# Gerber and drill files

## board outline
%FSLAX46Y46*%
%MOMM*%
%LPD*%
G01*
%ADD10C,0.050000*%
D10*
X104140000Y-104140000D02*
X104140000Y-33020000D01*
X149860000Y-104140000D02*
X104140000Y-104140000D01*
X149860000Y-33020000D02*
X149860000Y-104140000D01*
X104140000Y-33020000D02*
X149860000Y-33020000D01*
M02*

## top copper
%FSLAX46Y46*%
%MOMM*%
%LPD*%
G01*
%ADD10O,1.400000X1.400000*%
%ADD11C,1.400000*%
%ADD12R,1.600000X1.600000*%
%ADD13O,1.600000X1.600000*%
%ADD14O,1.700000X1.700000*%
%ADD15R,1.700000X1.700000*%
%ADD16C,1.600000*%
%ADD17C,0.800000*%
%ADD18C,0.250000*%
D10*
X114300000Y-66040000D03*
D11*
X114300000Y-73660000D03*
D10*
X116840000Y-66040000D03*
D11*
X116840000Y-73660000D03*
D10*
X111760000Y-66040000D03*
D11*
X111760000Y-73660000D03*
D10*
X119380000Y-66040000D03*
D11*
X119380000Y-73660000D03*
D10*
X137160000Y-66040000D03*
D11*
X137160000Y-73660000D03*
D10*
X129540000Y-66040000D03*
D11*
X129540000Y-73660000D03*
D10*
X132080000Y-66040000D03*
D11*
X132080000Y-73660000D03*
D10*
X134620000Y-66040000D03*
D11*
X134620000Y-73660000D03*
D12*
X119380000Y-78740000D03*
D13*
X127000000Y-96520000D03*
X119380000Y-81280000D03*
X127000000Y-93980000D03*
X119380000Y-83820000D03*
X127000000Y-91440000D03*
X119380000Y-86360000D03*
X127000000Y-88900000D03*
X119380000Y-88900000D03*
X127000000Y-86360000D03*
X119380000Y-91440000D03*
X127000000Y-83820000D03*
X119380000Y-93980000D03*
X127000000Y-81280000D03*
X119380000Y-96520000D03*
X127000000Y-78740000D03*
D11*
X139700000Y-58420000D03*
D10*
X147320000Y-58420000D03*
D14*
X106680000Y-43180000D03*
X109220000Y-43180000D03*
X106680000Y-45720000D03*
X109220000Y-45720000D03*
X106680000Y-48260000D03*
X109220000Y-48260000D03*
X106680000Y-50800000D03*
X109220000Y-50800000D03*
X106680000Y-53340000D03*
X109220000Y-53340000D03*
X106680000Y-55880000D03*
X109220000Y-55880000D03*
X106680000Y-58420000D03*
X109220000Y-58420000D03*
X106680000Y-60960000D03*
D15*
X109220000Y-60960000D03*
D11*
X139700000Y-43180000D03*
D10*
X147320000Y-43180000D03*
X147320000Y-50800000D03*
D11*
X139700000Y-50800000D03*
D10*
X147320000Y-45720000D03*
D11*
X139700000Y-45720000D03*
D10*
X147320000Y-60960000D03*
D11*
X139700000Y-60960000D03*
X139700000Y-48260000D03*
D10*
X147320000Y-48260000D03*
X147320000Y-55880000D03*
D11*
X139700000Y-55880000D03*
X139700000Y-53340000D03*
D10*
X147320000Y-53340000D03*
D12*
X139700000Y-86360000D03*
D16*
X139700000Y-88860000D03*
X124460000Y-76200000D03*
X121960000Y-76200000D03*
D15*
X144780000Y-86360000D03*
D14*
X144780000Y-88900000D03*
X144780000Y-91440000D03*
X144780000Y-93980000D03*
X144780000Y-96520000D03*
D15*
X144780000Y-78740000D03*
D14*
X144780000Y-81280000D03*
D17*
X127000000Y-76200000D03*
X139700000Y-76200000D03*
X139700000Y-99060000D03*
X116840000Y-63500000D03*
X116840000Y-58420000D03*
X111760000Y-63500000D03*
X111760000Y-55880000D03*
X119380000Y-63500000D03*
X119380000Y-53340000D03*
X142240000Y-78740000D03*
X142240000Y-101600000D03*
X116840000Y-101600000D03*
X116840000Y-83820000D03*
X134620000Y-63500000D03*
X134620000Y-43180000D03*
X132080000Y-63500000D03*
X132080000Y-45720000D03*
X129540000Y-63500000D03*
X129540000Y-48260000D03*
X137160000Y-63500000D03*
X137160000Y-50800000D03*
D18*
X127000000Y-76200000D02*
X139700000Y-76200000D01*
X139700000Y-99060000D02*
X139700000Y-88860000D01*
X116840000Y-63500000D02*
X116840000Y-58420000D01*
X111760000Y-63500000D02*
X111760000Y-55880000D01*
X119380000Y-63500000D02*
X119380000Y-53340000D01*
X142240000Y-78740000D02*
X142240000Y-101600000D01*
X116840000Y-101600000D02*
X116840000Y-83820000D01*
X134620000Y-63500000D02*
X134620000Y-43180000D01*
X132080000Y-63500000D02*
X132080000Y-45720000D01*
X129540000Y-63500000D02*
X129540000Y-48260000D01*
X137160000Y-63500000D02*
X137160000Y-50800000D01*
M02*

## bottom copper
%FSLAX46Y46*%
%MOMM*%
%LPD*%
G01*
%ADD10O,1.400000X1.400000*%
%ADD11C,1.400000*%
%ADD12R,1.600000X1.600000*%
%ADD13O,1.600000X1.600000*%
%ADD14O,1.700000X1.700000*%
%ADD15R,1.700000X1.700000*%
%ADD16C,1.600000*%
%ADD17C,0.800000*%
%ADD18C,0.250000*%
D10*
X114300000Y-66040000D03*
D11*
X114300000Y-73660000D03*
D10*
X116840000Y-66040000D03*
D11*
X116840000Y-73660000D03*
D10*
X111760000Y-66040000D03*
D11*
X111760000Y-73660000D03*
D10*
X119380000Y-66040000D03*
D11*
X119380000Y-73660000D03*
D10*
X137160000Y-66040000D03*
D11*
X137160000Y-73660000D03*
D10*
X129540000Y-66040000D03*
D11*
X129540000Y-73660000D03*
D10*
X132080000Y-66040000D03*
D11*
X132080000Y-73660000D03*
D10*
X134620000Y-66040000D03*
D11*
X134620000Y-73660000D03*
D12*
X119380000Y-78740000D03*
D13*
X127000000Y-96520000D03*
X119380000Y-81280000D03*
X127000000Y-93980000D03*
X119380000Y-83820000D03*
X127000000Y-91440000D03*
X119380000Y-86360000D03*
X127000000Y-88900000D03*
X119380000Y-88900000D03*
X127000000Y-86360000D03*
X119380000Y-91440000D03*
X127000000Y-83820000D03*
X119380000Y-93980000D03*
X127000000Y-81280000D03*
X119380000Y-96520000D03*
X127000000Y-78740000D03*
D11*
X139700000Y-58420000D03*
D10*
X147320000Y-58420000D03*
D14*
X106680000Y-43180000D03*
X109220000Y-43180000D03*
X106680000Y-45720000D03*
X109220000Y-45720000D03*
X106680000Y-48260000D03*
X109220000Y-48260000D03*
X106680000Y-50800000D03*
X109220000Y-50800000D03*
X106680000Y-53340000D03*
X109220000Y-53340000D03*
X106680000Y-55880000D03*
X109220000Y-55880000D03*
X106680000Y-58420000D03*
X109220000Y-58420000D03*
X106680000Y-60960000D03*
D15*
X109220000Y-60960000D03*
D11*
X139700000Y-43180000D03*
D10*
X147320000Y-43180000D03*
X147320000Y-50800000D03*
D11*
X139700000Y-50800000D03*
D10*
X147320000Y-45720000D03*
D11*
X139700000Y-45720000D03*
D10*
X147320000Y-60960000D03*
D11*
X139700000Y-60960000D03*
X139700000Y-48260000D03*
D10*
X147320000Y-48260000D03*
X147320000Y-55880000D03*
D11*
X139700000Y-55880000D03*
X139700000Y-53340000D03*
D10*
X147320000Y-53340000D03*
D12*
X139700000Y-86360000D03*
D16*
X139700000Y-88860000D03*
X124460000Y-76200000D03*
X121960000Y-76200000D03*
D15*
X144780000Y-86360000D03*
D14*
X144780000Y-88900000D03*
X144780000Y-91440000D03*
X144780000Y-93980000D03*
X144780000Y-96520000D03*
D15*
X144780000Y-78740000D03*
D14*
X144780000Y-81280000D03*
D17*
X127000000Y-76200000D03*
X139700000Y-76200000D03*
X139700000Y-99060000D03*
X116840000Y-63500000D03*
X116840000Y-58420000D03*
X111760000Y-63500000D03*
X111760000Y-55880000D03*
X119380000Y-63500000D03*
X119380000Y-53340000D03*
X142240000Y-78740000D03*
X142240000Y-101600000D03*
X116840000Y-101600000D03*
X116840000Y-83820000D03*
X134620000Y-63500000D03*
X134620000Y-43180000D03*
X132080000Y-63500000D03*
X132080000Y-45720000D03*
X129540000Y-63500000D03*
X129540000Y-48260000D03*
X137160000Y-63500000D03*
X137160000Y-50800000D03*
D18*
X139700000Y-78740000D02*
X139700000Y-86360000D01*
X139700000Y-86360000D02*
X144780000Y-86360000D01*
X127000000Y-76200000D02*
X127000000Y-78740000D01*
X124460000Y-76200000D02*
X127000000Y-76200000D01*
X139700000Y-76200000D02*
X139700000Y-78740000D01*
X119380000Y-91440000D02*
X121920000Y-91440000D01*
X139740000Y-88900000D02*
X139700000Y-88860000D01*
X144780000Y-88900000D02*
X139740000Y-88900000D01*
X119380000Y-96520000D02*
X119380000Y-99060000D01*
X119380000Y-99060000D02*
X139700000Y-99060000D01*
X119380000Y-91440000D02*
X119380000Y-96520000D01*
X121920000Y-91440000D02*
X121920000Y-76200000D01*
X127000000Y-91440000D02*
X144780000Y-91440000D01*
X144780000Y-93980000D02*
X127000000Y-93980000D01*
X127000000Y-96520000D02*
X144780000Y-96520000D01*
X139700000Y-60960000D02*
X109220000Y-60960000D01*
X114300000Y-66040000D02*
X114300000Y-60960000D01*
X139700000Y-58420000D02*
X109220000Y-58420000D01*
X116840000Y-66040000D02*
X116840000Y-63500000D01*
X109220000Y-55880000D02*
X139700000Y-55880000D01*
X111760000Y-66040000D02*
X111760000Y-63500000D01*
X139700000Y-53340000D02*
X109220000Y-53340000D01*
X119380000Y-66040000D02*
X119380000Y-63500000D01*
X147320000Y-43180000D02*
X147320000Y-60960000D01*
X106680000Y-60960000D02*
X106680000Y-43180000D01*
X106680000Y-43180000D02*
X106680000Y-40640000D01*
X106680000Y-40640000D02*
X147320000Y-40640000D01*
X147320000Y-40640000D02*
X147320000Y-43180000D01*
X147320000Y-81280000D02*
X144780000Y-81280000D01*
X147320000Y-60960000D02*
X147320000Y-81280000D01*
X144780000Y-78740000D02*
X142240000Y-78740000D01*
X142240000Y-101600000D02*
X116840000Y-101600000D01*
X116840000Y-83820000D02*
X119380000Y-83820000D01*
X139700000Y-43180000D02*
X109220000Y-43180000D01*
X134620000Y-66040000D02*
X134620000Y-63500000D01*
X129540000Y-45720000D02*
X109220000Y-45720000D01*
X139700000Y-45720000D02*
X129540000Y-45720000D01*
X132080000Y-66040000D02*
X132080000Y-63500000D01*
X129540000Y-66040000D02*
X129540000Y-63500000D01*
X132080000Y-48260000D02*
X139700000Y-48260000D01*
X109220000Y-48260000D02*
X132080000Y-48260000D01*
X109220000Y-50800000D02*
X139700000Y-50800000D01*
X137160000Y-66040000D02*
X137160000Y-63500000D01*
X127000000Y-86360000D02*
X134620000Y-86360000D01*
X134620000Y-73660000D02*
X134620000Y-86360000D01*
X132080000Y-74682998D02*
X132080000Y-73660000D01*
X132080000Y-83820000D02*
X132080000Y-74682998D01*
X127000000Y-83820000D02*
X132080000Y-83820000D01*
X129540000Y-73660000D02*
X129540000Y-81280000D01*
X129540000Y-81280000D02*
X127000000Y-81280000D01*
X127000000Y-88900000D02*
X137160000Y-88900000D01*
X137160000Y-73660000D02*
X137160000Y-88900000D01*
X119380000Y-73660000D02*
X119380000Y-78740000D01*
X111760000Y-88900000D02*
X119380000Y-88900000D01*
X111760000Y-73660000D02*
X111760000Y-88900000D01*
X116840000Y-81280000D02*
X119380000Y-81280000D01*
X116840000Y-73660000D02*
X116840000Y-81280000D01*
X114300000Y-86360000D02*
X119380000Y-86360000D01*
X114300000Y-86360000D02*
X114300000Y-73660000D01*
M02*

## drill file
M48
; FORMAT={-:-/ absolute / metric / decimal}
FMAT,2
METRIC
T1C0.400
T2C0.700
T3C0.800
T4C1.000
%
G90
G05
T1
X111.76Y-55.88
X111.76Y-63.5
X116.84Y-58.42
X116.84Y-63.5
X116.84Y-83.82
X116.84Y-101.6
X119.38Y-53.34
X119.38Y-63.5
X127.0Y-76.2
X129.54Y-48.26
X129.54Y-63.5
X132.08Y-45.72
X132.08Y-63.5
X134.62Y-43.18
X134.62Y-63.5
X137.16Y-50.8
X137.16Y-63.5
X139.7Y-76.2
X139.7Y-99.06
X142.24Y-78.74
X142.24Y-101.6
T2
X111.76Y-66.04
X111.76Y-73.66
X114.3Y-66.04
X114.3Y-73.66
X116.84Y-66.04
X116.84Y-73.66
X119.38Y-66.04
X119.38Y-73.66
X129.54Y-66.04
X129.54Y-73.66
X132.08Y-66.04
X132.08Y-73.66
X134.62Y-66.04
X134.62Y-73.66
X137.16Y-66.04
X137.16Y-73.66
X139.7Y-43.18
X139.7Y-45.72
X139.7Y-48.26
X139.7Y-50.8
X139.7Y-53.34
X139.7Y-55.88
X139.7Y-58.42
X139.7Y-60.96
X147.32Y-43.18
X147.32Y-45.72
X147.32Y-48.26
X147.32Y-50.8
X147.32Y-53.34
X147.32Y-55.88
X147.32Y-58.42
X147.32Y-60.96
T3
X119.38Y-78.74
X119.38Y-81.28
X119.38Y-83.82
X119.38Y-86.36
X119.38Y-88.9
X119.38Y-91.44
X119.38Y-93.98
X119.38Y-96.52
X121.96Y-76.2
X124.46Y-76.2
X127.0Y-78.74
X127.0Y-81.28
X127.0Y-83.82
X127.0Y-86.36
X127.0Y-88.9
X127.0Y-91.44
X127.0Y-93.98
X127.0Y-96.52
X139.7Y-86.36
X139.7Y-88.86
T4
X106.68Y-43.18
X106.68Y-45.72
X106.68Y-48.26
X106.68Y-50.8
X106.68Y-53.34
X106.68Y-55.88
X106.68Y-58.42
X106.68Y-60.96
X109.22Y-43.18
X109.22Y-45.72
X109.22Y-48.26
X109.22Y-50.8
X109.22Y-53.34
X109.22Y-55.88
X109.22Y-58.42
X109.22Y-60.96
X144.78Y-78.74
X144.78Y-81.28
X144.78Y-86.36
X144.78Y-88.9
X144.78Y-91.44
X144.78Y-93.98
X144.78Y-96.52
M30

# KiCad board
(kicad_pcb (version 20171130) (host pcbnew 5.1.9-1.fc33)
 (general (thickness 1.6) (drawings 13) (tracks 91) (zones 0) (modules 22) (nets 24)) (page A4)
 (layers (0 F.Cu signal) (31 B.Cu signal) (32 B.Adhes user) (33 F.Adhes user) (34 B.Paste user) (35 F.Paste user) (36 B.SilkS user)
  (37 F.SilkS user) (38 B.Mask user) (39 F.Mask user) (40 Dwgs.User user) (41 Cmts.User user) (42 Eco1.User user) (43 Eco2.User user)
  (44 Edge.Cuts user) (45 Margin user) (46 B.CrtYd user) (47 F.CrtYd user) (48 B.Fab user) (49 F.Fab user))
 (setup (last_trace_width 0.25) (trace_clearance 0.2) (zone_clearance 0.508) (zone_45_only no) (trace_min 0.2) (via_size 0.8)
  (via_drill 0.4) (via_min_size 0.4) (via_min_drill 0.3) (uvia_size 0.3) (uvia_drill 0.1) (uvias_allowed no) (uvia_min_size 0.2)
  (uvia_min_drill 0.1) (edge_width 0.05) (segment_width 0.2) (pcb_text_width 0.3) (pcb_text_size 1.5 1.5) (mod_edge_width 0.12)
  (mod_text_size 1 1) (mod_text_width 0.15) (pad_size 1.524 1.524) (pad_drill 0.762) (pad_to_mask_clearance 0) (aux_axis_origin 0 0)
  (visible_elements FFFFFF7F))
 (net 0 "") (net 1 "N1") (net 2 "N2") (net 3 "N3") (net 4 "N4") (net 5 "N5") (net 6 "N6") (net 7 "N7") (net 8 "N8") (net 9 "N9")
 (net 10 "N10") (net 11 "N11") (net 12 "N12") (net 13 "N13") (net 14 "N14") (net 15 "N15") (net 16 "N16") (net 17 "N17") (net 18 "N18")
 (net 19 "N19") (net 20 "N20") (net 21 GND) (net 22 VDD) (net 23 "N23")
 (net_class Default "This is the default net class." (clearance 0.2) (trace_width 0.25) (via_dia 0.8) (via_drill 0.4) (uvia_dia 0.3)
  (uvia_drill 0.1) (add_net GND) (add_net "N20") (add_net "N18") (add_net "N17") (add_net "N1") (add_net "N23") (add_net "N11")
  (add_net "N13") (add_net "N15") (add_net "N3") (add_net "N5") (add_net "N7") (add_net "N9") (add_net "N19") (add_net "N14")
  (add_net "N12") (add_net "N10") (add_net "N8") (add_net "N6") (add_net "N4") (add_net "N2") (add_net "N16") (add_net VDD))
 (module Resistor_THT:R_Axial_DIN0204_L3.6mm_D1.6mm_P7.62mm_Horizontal (layer F.Cu) (at 114.3 73.66 90)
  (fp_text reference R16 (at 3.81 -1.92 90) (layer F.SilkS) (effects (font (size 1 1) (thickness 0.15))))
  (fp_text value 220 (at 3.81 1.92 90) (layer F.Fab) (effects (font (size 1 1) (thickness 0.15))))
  (pad 2 thru_hole oval (at 7.62 0 90) (size 1.4 1.4) (drill 0.7) (layers *.Cu *.Mask) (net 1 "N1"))
  (pad 1 thru_hole circle (at 0 0 90) (size 1.4 1.4) (drill 0.7) (layers *.Cu *.Mask) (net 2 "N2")))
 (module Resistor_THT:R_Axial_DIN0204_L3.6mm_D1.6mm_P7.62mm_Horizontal (layer F.Cu) (at 116.84 73.66 90)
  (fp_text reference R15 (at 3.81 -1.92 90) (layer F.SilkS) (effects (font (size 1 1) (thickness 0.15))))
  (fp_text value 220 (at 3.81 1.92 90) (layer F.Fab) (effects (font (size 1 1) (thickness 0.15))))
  (pad 2 thru_hole oval (at 7.62 0 90) (size 1.4 1.4) (drill 0.7) (layers *.Cu *.Mask) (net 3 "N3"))
  (pad 1 thru_hole circle (at 0 0 90) (size 1.4 1.4) (drill 0.7) (layers *.Cu *.Mask) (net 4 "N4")))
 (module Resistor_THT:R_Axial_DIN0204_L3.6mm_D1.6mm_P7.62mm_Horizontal (layer F.Cu) (at 111.76 73.66 90)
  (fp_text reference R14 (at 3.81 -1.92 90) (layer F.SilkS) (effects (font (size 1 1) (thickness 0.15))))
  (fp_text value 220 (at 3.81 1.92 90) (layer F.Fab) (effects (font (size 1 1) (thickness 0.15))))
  (pad 2 thru_hole oval (at 7.62 0 90) (size 1.4 1.4) (drill 0.7) (layers *.Cu *.Mask) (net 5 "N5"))
  (pad 1 thru_hole circle (at 0 0 90) (size 1.4 1.4) (drill 0.7) (layers *.Cu *.Mask) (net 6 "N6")))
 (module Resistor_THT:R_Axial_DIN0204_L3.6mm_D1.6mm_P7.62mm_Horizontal (layer F.Cu) (at 119.38 73.66 90)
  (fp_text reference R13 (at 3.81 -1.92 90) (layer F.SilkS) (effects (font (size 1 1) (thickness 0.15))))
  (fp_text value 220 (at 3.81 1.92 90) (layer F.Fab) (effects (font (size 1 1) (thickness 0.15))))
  (pad 2 thru_hole oval (at 7.62 0 90) (size 1.4 1.4) (drill 0.7) (layers *.Cu *.Mask) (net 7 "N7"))
  (pad 1 thru_hole circle (at 0 0 90) (size 1.4 1.4) (drill 0.7) (layers *.Cu *.Mask) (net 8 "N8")))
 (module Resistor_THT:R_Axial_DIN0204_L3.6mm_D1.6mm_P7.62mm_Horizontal (layer F.Cu) (at 137.16 73.66 90)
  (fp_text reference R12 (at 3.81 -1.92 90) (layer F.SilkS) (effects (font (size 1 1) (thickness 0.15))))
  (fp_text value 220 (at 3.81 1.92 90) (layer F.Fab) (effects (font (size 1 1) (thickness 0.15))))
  (pad 2 thru_hole oval (at 7.62 0 90) (size 1.4 1.4) (drill 0.7) (layers *.Cu *.Mask) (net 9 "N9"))
  (pad 1 thru_hole circle (at 0 0 90) (size 1.4 1.4) (drill 0.7) (layers *.Cu *.Mask) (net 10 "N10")))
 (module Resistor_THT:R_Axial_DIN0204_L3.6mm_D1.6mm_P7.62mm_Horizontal (layer F.Cu) (at 129.54 73.66 90)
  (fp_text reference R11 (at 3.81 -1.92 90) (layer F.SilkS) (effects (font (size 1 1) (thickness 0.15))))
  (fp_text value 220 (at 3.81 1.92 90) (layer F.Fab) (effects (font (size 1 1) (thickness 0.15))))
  (pad 2 thru_hole oval (at 7.62 0 90) (size 1.4 1.4) (drill 0.7) (layers *.Cu *.Mask) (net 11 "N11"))
  (pad 1 thru_hole circle (at 0 0 90) (size 1.4 1.4) (drill 0.7) (layers *.Cu *.Mask) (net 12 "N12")))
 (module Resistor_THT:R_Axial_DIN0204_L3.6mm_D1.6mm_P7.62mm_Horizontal (layer F.Cu) (at 132.08 73.66 90)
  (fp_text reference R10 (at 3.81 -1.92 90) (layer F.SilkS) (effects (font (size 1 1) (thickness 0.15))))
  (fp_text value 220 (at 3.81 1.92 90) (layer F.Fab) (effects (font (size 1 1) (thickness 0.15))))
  (pad 2 thru_hole oval (at 7.62 0 90) (size 1.4 1.4) (drill 0.7) (layers *.Cu *.Mask) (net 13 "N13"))
  (pad 1 thru_hole circle (at 0 0 90) (size 1.4 1.4) (drill 0.7) (layers *.Cu *.Mask) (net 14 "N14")))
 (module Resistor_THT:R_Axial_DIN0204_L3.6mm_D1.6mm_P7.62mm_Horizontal (layer F.Cu) (at 134.62 73.66 90)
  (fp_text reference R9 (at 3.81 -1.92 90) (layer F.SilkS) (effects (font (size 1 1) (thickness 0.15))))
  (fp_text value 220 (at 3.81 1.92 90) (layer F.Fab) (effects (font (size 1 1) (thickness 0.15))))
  (pad 2 thru_hole oval (at 7.62 0 90) (size 1.4 1.4) (drill 0.7) (layers *.Cu *.Mask) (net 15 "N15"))
  (pad 1 thru_hole circle (at 0 0 90) (size 1.4 1.4) (drill 0.7) (layers *.Cu *.Mask) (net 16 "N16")))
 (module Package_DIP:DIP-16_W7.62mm (layer F.Cu) (at 119.38 78.74)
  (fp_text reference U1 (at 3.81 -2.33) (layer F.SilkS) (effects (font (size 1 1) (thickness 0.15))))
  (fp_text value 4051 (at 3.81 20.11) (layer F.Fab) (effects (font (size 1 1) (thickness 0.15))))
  (pad 1 thru_hole rect (at 0 0) (size 1.6 1.6) (drill 0.8) (layers *.Cu *.Mask) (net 8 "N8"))
  (pad 9 thru_hole oval (at 7.62 17.78) (size 1.6 1.6) (drill 0.8) (layers *.Cu *.Mask) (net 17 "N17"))
  (pad 2 thru_hole oval (at 0 2.54) (size 1.6 1.6) (drill 0.8) (layers *.Cu *.Mask) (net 4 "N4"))
  (pad 10 thru_hole oval (at 7.62 15.24) (size 1.6 1.6) (drill 0.8) (layers *.Cu *.Mask) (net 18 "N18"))
  (pad 3 thru_hole oval (at 0 5.08) (size 1.6 1.6) (drill 0.8) (layers *.Cu *.Mask) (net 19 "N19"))
  (pad 11 thru_hole oval (at 7.62 12.7) (size 1.6 1.6) (drill 0.8) (layers *.Cu *.Mask) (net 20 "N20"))
  (pad 4 thru_hole oval (at 0 7.62) (size 1.6 1.6) (drill 0.8) (layers *.Cu *.Mask) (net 2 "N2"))
  (pad 12 thru_hole oval (at 7.62 10.16) (size 1.6 1.6) (drill 0.8) (layers *.Cu *.Mask) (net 10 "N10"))
  (pad 5 thru_hole oval (at 0 10.16) (size 1.6 1.6) (drill 0.8) (layers *.Cu *.Mask) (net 6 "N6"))
  (pad 13 thru_hole oval (at 7.62 7.62) (size 1.6 1.6) (drill 0.8) (layers *.Cu *.Mask) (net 16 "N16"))
  (pad 6 thru_hole oval (at 0 12.7) (size 1.6 1.6) (drill 0.8) (layers *.Cu *.Mask) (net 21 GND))
  (pad 14 thru_hole oval (at 7.62 5.08) (size 1.6 1.6) (drill 0.8) (layers *.Cu *.Mask) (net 14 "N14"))
  (pad 7 thru_hole oval (at 0 15.24) (size 1.6 1.6) (drill 0.8) (layers *.Cu *.Mask) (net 21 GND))
  (pad 15 thru_hole oval (at 7.62 2.54) (size 1.6 1.6) (drill 0.8) (layers *.Cu *.Mask) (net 12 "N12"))
  (pad 8 thru_hole oval (at 0 17.78) (size 1.6 1.6) (drill 0.8) (layers *.Cu *.Mask) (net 21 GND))
  (pad 16 thru_hole oval (at 7.62 0) (size 1.6 1.6) (drill 0.8) (layers *.Cu *.Mask) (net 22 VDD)))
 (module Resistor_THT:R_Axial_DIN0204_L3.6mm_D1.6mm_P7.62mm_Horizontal (layer F.Cu) (at 139.7 58.42)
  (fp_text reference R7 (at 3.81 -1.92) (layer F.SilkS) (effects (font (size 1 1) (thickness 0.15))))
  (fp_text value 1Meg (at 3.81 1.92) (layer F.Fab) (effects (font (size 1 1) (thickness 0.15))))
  (pad 1 thru_hole circle (at 0 0) (size 1.4 1.4) (drill 0.7) (layers *.Cu *.Mask) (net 3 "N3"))
  (pad 2 thru_hole oval (at 7.62 0) (size 1.4 1.4) (drill 0.7) (layers *.Cu *.Mask) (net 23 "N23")))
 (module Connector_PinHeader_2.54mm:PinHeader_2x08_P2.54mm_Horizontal (layer F.Cu) (at 109.22 60.96 180)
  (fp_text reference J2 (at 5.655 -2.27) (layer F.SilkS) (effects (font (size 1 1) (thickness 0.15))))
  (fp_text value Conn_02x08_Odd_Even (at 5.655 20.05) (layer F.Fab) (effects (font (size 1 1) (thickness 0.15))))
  (pad 16 thru_hole oval (at 2.54 17.78 180) (size 1.7 1.7) (drill 1) (layers *.Cu *.Mask) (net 23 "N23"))
  (pad 15 thru_hole oval (at 0 17.78 180) (size 1.7 1.7) (drill 1) (layers *.Cu *.Mask) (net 15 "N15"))
  (pad 14 thru_hole oval (at 2.54 15.24 180) (size 1.7 1.7) (drill 1) (layers *.Cu *.Mask) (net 23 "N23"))
  (pad 13 thru_hole oval (at 0 15.24 180) (size 1.7 1.7) (drill 1) (layers *.Cu *.Mask) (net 13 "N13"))
  (pad 12 thru_hole oval (at 2.54 12.7 180) (size 1.7 1.7) (drill 1) (layers *.Cu *.Mask) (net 23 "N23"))
  (pad 11 thru_hole oval (at 0 12.7 180) (size 1.7 1.7) (drill 1) (layers *.Cu *.Mask) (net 11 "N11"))
  (pad 10 thru_hole oval (at 2.54 10.16 180) (size 1.7 1.7) (drill 1) (layers *.Cu *.Mask) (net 23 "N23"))
  (pad 9 thru_hole oval (at 0 10.16 180) (size 1.7 1.7) (drill 1) (layers *.Cu *.Mask) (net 9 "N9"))
  (pad 8 thru_hole oval (at 2.54 7.62 180) (size 1.7 1.7) (drill 1) (layers *.Cu *.Mask) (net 23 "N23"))
  (pad 7 thru_hole oval (at 0 7.62 180) (size 1.7 1.7) (drill 1) (layers *.Cu *.Mask) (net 7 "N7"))
  (pad 6 thru_hole oval (at 2.54 5.08 180) (size 1.7 1.7) (drill 1) (layers *.Cu *.Mask) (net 23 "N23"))
  (pad 5 thru_hole oval (at 0 5.08 180) (size 1.7 1.7) (drill 1) (layers *.Cu *.Mask) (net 5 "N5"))
  (pad 4 thru_hole oval (at 2.54 2.54 180) (size 1.7 1.7) (drill 1) (layers *.Cu *.Mask) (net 23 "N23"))
  (pad 3 thru_hole oval (at 0 2.54 180) (size 1.7 1.7) (drill 1) (layers *.Cu *.Mask) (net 3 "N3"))
  (pad 2 thru_hole oval (at 2.54 0 180) (size 1.7 1.7) (drill 1) (layers *.Cu *.Mask) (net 23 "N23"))
  (pad 1 thru_hole rect (at 0 0 180) (size 1.7 1.7) (drill 1) (layers *.Cu *.Mask) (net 1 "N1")))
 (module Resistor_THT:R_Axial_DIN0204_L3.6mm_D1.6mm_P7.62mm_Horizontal (layer F.Cu) (at 139.7 43.18)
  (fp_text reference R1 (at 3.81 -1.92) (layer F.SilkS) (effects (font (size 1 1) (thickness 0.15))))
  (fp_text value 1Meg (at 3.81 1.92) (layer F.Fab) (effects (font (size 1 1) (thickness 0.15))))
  (pad 1 thru_hole circle (at 0 0) (size 1.4 1.4) (drill 0.7) (layers *.Cu *.Mask) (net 15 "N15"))
  (pad 2 thru_hole oval (at 7.62 0) (size 1.4 1.4) (drill 0.7) (layers *.Cu *.Mask) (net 23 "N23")))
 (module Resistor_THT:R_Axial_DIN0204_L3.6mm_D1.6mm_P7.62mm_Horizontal (layer F.Cu) (at 139.7 50.8)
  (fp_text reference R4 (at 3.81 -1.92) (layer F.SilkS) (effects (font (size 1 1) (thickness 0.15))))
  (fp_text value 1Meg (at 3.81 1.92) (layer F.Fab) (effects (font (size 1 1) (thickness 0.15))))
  (pad 2 thru_hole oval (at 7.62 0) (size 1.4 1.4) (drill 0.7) (layers *.Cu *.Mask) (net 23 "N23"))
  (pad 1 thru_hole circle (at 0 0) (size 1.4 1.4) (drill 0.7) (layers *.Cu *.Mask) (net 9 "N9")))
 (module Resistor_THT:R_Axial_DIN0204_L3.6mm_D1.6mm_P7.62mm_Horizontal (layer F.Cu) (at 139.7 45.72)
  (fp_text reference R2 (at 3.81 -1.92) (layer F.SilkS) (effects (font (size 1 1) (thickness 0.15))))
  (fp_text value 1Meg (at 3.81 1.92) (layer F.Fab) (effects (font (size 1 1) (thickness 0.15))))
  (pad 2 thru_hole oval (at 7.62 0) (size 1.4 1.4) (drill 0.7) (layers *.Cu *.Mask) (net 23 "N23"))
  (pad 1 thru_hole circle (at 0 0) (size 1.4 1.4) (drill 0.7) (layers *.Cu *.Mask) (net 13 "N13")))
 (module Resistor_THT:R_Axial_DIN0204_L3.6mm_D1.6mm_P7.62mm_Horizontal (layer F.Cu) (at 139.7 60.96)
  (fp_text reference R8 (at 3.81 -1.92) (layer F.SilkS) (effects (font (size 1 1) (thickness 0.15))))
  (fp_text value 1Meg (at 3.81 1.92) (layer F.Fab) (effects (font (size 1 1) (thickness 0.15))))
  (pad 2 thru_hole oval (at 7.62 0) (size 1.4 1.4) (drill 0.7) (layers *.Cu *.Mask) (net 23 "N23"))
  (pad 1 thru_hole circle (at 0 0) (size 1.4 1.4) (drill 0.7) (layers *.Cu *.Mask) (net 1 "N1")))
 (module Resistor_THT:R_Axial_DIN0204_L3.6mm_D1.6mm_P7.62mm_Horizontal (layer F.Cu) (at 139.7 48.26)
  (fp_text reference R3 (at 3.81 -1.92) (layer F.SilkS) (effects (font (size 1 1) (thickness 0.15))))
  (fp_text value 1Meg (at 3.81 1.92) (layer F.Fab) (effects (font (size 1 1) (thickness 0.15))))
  (pad 1 thru_hole circle (at 0 0) (size 1.4 1.4) (drill 0.7) (layers *.Cu *.Mask) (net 11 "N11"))
  (pad 2 thru_hole oval (at 7.62 0) (size 1.4 1.4) (drill 0.7) (layers *.Cu *.Mask) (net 23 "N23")))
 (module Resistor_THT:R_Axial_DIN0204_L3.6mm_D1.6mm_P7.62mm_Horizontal (layer F.Cu) (at 139.7 55.88)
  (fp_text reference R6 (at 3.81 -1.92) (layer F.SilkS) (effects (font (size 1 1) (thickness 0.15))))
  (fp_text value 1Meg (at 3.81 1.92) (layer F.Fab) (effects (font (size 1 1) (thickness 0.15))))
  (pad 2 thru_hole oval (at 7.62 0) (size 1.4 1.4) (drill 0.7) (layers *.Cu *.Mask) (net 23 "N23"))
  (pad 1 thru_hole circle (at 0 0) (size 1.4 1.4) (drill 0.7) (layers *.Cu *.Mask) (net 5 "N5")))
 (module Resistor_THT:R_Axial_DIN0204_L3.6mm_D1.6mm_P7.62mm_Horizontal (layer F.Cu) (at 139.7 53.34)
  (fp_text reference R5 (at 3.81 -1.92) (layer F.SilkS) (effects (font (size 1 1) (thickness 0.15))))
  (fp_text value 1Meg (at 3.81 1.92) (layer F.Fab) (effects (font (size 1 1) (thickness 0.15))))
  (pad 1 thru_hole circle (at 0 0) (size 1.4 1.4) (drill 0.7) (layers *.Cu *.Mask) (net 7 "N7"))
  (pad 2 thru_hole oval (at 7.62 0) (size 1.4 1.4) (drill 0.7) (layers *.Cu *.Mask) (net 23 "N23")))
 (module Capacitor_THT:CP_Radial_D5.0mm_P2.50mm (layer F.Cu) (at 139.7 86.36 270)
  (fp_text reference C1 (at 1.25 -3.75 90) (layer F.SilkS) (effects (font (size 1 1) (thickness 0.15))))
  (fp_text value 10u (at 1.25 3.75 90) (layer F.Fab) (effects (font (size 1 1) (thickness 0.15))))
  (pad 1 thru_hole rect (at 0 0 270) (size 1.6 1.6) (drill 0.8) (layers *.Cu *.Mask) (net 22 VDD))
  (pad 2 thru_hole circle (at 2.5 0 270) (size 1.6 1.6) (drill 0.8) (layers *.Cu *.Mask) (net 21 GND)))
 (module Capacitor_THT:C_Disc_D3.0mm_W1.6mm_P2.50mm (layer F.Cu) (at 124.46 76.2 180)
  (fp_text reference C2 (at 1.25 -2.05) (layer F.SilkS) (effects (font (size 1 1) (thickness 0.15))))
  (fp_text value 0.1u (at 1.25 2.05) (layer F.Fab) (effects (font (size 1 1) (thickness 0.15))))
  (pad 1 thru_hole circle (at 0 0 180) (size 1.6 1.6) (drill 0.8) (layers *.Cu *.Mask) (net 22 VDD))
  (pad 2 thru_hole circle (at 2.5 0 180) (size 1.6 1.6) (drill 0.8) (layers *.Cu *.Mask) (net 21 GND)))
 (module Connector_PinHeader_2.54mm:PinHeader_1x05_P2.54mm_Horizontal (layer F.Cu) (at 144.78 86.36)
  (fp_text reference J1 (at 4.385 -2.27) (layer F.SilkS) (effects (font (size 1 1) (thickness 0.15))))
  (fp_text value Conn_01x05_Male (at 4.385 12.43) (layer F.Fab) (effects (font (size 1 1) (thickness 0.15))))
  (pad 1 thru_hole rect (at 0 0) (size 1.7 1.7) (drill 1) (layers *.Cu *.Mask) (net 22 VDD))
  (pad 2 thru_hole oval (at 0 2.54) (size 1.7 1.7) (drill 1) (layers *.Cu *.Mask) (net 21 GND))
  (pad 3 thru_hole oval (at 0 5.08) (size 1.7 1.7) (drill 1) (layers *.Cu *.Mask) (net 20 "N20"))
  (pad 4 thru_hole oval (at 0 7.62) (size 1.7 1.7) (drill 1) (layers *.Cu *.Mask) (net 18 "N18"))
  (pad 5 thru_hole oval (at 0 10.16) (size 1.7 1.7) (drill 1) (layers *.Cu *.Mask) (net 17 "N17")))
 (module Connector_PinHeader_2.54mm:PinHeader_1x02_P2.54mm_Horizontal (layer F.Cu) (at 144.78 78.74)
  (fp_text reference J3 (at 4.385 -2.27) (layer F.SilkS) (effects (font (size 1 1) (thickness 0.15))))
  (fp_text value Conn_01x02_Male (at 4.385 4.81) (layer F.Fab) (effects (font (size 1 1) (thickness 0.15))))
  (pad 1 thru_hole rect (at 0 0) (size 1.7 1.7) (drill 1) (layers *.Cu *.Mask) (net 19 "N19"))
  (pad 2 thru_hole oval (at 0 2.54) (size 1.7 1.7) (drill 1) (layers *.Cu *.Mask) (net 23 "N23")))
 (gr_line (start 104.14 104.14) (end 104.14 33.02) (layer Edge.Cuts) (width 0.05))
 (gr_line (start 149.86 104.14) (end 104.14 104.14) (layer Edge.Cuts) (width 0.05))
 (gr_line (start 149.86 33.02) (end 149.86 104.14) (layer Edge.Cuts) (width 0.05))
 (gr_line (start 104.14 33.02) (end 149.86 33.02) (layer Edge.Cuts) (width 0.05))
 (segment (start 139.7 78.74) (end 139.7 86.36) (width 0.25) (layer B.Cu) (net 22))
 (segment (start 139.7 86.36) (end 144.78 86.36) (width 0.25) (layer B.Cu) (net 22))
 (segment (start 127 76.2) (end 127 78.74) (width 0.25) (layer B.Cu) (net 22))
 (via (at 127 76.2) (size 0.8) (drill 0.4) (layers F.Cu B.Cu) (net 22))
 (segment (start 124.46 76.2) (end 127 76.2) (width 0.25) (layer B.Cu) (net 22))
 (via (at 139.7 76.2) (size 0.8) (drill 0.4) (layers F.Cu B.Cu) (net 22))
 (segment (start 127 76.2) (end 139.7 76.2) (width 0.25) (layer F.Cu) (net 22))
 (segment (start 139.7 76.2) (end 139.7 78.74) (width 0.25) (layer B.Cu) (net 22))
 (segment (start 119.38 91.44) (end 121.92 91.44) (width 0.25) (layer B.Cu) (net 21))
 (segment (start 139.74 88.9) (end 139.7 88.86) (width 0.25) (layer B.Cu) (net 21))
 (segment (start 144.78 88.9) (end 139.74 88.9) (width 0.25) (layer B.Cu) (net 21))
 (segment (start 119.38 96.52) (end 119.38 99.06) (width 0.25) (layer B.Cu) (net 21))
 (via (at 139.7 99.06) (size 0.8) (drill 0.4) (layers F.Cu B.Cu) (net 21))
 (segment (start 119.38 99.06) (end 139.7 99.06) (width 0.25) (layer B.Cu) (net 21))
 (segment (start 139.7 99.06) (end 139.7 88.86) (width 0.25) (layer F.Cu) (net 21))
 (segment (start 119.38 91.44) (end 119.38 96.52) (width 0.25) (layer B.Cu) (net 21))
 (segment (start 121.92 91.44) (end 121.92 76.2) (width 0.25) (layer B.Cu) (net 21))
 (segment (start 127 91.44) (end 144.78 91.44) (width 0.25) (layer B.Cu) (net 20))
 (segment (start 144.78 93.98) (end 127 93.98) (width 0.25) (layer B.Cu) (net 18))
 (segment (start 127 96.52) (end 144.78 96.52) (width 0.25) (layer B.Cu) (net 17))
 (segment (start 139.7 60.96) (end 109.22 60.96) (width 0.25) (layer B.Cu) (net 1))
 (segment (start 114.3 66.04) (end 114.3 60.96) (width 0.25) (layer B.Cu) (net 1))
 (segment (start 139.7 58.42) (end 109.22 58.42) (width 0.25) (layer B.Cu) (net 3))
 (via (at 116.84 63.5) (size 0.8) (drill 0.4) (layers F.Cu B.Cu) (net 3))
 (segment (start 116.84 66.04) (end 116.84 63.5) (width 0.25) (layer B.Cu) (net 3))
 (via (at 116.84 58.42) (size 0.8) (drill 0.4) (layers F.Cu B.Cu) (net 3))
 (segment (start 116.84 63.5) (end 116.84 58.42) (width 0.25) (layer F.Cu) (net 3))
 (segment (start 109.22 55.88) (end 139.7 55.88) (width 0.25) (layer B.Cu) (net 5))
 (via (at 111.76 63.5) (size 0.8) (drill 0.4) (layers F.Cu B.Cu) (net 5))
 (segment (start 111.76 66.04) (end 111.76 63.5) (width 0.25) (layer B.Cu) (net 5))
 (segment (start 111.76 63.5) (end 111.76 55.88) (width 0.25) (layer F.Cu) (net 5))
 (via (at 111.76 55.88) (size 0.8) (drill 0.4) (layers F.Cu B.Cu) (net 5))
 (segment (start 139.7 53.34) (end 109.22 53.34) (width 0.25) (layer B.Cu) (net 7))
 (via (at 119.38 63.5) (size 0.8) (drill 0.4) (layers F.Cu B.Cu) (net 7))
 (segment (start 119.38 66.04) (end 119.38 63.5) (width 0.25) (layer B.Cu) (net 7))
 (via (at 119.38 53.34) (size 0.8) (drill 0.4) (layers F.Cu B.Cu) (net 7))
 (segment (start 119.38 63.5) (end 119.38 53.34) (width 0.25) (layer F.Cu) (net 7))
 (segment (start 147.32 43.18) (end 147.32 60.96) (width 0.25) (layer B.Cu) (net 23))
 (segment (start 106.68 60.96) (end 106.68 43.18) (width 0.25) (layer B.Cu) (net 23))
 (segment (start 106.68 43.18) (end 106.68 40.64) (width 0.25) (layer B.Cu) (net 23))
 (segment (start 106.68 40.64) (end 147.32 40.64) (width 0.25) (layer B.Cu) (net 23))
 (segment (start 147.32 40.64) (end 147.32 43.18) (width 0.25) (layer B.Cu) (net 23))
 (segment (start 147.32 81.28) (end 144.78 81.28) (width 0.25) (layer B.Cu) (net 23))
 (segment (start 147.32 60.96) (end 147.32 81.28) (width 0.25) (layer B.Cu) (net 23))
 (via (at 142.24 78.74) (size 0.8) (drill 0.4) (layers F.Cu B.Cu) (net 19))
 (segment (start 144.78 78.74) (end 142.24 78.74) (width 0.25) (layer B.Cu) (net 19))
 (via (at 142.24 101.6) (size 0.8) (drill 0.4) (layers F.Cu B.Cu) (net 19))
 (segment (start 142.24 78.74) (end 142.24 101.6) (width 0.25) (layer F.Cu) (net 19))
 (via (at 116.84 101.6) (size 0.8) (drill 0.4) (layers F.Cu B.Cu) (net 19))
 (segment (start 142.24 101.6) (end 116.84 101.6) (width 0.25) (layer B.Cu) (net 19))
 (via (at 116.84 83.82) (size 0.8) (drill 0.4) (layers F.Cu B.Cu) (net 19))
 (segment (start 116.84 101.6) (end 116.84 83.82) (width 0.25) (layer F.Cu) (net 19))
 (segment (start 116.84 83.82) (end 119.38 83.82) (width 0.25) (layer B.Cu) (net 19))
 (segment (start 139.7 43.18) (end 109.22 43.18) (width 0.25) (layer B.Cu) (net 15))
 (via (at 134.62 63.5) (size 0.8) (drill 0.4) (layers F.Cu B.Cu) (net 15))
 (segment (start 134.62 66.04) (end 134.62 63.5) (width 0.25) (layer B.Cu) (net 15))
 (via (at 134.62 43.18) (size 0.8) (drill 0.4) (layers F.Cu B.Cu) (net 15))
 (segment (start 134.62 63.5) (end 134.62 43.18) (width 0.25) (layer F.Cu) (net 15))
 (segment (start 129.54 45.72) (end 109.22 45.72) (width 0.25) (layer B.Cu) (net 13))
 (segment (start 139.7 45.72) (end 129.54 45.72) (width 0.25) (layer B.Cu) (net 13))
 (via (at 132.08 63.5) (size 0.8) (drill 0.4) (layers F.Cu B.Cu) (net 13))
 (segment (start 132.08 66.04) (end 132.08 63.5) (width 0.25) (layer B.Cu) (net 13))
 (via (at 132.08 45.72) (size 0.8) (drill 0.4) (layers F.Cu B.Cu) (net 13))
 (segment (start 132.08 63.5) (end 132.08 45.72) (width 0.25) (layer F.Cu) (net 13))
 (via (at 129.54 63.5) (size 0.8) (drill 0.4) (layers F.Cu B.Cu) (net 11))
 (segment (start 129.54 66.04) (end 129.54 63.5) (width 0.25) (layer B.Cu) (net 11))
 (segment (start 132.08 48.26) (end 139.7 48.26) (width 0.25) (layer B.Cu) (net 11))
 (segment (start 109.22 48.26) (end 132.08 48.26) (width 0.25) (layer B.Cu) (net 11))
 (via (at 129.54 48.26) (size 0.8) (drill 0.4) (layers F.Cu B.Cu) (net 11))
 (segment (start 129.54 63.5) (end 129.54 48.26) (width 0.25) (layer F.Cu) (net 11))
 (segment (start 109.22 50.8) (end 139.7 50.8) (width 0.25) (layer B.Cu) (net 9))
 (via (at 137.16 63.5) (size 0.8) (drill 0.4) (layers F.Cu B.Cu) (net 9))
 (segment (start 137.16 66.04) (end 137.16 63.5) (width 0.25) (layer B.Cu) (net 9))
 (via (at 137.16 50.8) (size 0.8) (drill 0.4) (layers F.Cu B.Cu) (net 9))
 (segment (start 137.16 63.5) (end 137.16 50.8) (width 0.25) (layer F.Cu) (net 9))
 (segment (start 127 86.36) (end 134.62 86.36) (width 0.25) (layer B.Cu) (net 16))
 (segment (start 134.62 73.66) (end 134.62 86.36) (width 0.25) (layer B.Cu) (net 16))
 (segment (start 132.08 74.682998) (end 132.08 73.66) (width 0.25) (layer B.Cu) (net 14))
 (segment (start 132.08 83.82) (end 132.08 74.682998) (width 0.25) (layer B.Cu) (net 14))
 (segment (start 127 83.82) (end 132.08 83.82) (width 0.25) (layer B.Cu) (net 14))
 (segment (start 129.54 73.66) (end 129.54 81.28) (width 0.25) (layer B.Cu) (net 12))
 (segment (start 129.54 81.28) (end 127 81.28) (width 0.25) (layer B.Cu) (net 12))
 (segment (start 127 88.9) (end 137.16 88.9) (width 0.25) (layer B.Cu) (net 10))
 (segment (start 137.16 73.66) (end 137.16 88.9) (width 0.25) (layer B.Cu) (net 10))
 (segment (start 119.38 73.66) (end 119.38 78.74) (width 0.25) (layer B.Cu) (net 8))
 (segment (start 111.76 88.9) (end 119.38 88.9) (width 0.25) (layer B.Cu) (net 6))
 (segment (start 111.76 73.66) (end 111.76 88.9) (width 0.25) (layer B.Cu) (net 6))
 (segment (start 116.84 81.28) (end 119.38 81.28) (width 0.25) (layer B.Cu) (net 4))
 (segment (start 116.84 73.66) (end 116.84 81.28) (width 0.25) (layer B.Cu) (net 4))
 (segment (start 114.3 86.36) (end 119.38 86.36) (width 0.25) (layer B.Cu) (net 2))
 (segment (start 114.3 86.36) (end 114.3 73.66) (width 0.25) (layer B.Cu) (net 2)))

